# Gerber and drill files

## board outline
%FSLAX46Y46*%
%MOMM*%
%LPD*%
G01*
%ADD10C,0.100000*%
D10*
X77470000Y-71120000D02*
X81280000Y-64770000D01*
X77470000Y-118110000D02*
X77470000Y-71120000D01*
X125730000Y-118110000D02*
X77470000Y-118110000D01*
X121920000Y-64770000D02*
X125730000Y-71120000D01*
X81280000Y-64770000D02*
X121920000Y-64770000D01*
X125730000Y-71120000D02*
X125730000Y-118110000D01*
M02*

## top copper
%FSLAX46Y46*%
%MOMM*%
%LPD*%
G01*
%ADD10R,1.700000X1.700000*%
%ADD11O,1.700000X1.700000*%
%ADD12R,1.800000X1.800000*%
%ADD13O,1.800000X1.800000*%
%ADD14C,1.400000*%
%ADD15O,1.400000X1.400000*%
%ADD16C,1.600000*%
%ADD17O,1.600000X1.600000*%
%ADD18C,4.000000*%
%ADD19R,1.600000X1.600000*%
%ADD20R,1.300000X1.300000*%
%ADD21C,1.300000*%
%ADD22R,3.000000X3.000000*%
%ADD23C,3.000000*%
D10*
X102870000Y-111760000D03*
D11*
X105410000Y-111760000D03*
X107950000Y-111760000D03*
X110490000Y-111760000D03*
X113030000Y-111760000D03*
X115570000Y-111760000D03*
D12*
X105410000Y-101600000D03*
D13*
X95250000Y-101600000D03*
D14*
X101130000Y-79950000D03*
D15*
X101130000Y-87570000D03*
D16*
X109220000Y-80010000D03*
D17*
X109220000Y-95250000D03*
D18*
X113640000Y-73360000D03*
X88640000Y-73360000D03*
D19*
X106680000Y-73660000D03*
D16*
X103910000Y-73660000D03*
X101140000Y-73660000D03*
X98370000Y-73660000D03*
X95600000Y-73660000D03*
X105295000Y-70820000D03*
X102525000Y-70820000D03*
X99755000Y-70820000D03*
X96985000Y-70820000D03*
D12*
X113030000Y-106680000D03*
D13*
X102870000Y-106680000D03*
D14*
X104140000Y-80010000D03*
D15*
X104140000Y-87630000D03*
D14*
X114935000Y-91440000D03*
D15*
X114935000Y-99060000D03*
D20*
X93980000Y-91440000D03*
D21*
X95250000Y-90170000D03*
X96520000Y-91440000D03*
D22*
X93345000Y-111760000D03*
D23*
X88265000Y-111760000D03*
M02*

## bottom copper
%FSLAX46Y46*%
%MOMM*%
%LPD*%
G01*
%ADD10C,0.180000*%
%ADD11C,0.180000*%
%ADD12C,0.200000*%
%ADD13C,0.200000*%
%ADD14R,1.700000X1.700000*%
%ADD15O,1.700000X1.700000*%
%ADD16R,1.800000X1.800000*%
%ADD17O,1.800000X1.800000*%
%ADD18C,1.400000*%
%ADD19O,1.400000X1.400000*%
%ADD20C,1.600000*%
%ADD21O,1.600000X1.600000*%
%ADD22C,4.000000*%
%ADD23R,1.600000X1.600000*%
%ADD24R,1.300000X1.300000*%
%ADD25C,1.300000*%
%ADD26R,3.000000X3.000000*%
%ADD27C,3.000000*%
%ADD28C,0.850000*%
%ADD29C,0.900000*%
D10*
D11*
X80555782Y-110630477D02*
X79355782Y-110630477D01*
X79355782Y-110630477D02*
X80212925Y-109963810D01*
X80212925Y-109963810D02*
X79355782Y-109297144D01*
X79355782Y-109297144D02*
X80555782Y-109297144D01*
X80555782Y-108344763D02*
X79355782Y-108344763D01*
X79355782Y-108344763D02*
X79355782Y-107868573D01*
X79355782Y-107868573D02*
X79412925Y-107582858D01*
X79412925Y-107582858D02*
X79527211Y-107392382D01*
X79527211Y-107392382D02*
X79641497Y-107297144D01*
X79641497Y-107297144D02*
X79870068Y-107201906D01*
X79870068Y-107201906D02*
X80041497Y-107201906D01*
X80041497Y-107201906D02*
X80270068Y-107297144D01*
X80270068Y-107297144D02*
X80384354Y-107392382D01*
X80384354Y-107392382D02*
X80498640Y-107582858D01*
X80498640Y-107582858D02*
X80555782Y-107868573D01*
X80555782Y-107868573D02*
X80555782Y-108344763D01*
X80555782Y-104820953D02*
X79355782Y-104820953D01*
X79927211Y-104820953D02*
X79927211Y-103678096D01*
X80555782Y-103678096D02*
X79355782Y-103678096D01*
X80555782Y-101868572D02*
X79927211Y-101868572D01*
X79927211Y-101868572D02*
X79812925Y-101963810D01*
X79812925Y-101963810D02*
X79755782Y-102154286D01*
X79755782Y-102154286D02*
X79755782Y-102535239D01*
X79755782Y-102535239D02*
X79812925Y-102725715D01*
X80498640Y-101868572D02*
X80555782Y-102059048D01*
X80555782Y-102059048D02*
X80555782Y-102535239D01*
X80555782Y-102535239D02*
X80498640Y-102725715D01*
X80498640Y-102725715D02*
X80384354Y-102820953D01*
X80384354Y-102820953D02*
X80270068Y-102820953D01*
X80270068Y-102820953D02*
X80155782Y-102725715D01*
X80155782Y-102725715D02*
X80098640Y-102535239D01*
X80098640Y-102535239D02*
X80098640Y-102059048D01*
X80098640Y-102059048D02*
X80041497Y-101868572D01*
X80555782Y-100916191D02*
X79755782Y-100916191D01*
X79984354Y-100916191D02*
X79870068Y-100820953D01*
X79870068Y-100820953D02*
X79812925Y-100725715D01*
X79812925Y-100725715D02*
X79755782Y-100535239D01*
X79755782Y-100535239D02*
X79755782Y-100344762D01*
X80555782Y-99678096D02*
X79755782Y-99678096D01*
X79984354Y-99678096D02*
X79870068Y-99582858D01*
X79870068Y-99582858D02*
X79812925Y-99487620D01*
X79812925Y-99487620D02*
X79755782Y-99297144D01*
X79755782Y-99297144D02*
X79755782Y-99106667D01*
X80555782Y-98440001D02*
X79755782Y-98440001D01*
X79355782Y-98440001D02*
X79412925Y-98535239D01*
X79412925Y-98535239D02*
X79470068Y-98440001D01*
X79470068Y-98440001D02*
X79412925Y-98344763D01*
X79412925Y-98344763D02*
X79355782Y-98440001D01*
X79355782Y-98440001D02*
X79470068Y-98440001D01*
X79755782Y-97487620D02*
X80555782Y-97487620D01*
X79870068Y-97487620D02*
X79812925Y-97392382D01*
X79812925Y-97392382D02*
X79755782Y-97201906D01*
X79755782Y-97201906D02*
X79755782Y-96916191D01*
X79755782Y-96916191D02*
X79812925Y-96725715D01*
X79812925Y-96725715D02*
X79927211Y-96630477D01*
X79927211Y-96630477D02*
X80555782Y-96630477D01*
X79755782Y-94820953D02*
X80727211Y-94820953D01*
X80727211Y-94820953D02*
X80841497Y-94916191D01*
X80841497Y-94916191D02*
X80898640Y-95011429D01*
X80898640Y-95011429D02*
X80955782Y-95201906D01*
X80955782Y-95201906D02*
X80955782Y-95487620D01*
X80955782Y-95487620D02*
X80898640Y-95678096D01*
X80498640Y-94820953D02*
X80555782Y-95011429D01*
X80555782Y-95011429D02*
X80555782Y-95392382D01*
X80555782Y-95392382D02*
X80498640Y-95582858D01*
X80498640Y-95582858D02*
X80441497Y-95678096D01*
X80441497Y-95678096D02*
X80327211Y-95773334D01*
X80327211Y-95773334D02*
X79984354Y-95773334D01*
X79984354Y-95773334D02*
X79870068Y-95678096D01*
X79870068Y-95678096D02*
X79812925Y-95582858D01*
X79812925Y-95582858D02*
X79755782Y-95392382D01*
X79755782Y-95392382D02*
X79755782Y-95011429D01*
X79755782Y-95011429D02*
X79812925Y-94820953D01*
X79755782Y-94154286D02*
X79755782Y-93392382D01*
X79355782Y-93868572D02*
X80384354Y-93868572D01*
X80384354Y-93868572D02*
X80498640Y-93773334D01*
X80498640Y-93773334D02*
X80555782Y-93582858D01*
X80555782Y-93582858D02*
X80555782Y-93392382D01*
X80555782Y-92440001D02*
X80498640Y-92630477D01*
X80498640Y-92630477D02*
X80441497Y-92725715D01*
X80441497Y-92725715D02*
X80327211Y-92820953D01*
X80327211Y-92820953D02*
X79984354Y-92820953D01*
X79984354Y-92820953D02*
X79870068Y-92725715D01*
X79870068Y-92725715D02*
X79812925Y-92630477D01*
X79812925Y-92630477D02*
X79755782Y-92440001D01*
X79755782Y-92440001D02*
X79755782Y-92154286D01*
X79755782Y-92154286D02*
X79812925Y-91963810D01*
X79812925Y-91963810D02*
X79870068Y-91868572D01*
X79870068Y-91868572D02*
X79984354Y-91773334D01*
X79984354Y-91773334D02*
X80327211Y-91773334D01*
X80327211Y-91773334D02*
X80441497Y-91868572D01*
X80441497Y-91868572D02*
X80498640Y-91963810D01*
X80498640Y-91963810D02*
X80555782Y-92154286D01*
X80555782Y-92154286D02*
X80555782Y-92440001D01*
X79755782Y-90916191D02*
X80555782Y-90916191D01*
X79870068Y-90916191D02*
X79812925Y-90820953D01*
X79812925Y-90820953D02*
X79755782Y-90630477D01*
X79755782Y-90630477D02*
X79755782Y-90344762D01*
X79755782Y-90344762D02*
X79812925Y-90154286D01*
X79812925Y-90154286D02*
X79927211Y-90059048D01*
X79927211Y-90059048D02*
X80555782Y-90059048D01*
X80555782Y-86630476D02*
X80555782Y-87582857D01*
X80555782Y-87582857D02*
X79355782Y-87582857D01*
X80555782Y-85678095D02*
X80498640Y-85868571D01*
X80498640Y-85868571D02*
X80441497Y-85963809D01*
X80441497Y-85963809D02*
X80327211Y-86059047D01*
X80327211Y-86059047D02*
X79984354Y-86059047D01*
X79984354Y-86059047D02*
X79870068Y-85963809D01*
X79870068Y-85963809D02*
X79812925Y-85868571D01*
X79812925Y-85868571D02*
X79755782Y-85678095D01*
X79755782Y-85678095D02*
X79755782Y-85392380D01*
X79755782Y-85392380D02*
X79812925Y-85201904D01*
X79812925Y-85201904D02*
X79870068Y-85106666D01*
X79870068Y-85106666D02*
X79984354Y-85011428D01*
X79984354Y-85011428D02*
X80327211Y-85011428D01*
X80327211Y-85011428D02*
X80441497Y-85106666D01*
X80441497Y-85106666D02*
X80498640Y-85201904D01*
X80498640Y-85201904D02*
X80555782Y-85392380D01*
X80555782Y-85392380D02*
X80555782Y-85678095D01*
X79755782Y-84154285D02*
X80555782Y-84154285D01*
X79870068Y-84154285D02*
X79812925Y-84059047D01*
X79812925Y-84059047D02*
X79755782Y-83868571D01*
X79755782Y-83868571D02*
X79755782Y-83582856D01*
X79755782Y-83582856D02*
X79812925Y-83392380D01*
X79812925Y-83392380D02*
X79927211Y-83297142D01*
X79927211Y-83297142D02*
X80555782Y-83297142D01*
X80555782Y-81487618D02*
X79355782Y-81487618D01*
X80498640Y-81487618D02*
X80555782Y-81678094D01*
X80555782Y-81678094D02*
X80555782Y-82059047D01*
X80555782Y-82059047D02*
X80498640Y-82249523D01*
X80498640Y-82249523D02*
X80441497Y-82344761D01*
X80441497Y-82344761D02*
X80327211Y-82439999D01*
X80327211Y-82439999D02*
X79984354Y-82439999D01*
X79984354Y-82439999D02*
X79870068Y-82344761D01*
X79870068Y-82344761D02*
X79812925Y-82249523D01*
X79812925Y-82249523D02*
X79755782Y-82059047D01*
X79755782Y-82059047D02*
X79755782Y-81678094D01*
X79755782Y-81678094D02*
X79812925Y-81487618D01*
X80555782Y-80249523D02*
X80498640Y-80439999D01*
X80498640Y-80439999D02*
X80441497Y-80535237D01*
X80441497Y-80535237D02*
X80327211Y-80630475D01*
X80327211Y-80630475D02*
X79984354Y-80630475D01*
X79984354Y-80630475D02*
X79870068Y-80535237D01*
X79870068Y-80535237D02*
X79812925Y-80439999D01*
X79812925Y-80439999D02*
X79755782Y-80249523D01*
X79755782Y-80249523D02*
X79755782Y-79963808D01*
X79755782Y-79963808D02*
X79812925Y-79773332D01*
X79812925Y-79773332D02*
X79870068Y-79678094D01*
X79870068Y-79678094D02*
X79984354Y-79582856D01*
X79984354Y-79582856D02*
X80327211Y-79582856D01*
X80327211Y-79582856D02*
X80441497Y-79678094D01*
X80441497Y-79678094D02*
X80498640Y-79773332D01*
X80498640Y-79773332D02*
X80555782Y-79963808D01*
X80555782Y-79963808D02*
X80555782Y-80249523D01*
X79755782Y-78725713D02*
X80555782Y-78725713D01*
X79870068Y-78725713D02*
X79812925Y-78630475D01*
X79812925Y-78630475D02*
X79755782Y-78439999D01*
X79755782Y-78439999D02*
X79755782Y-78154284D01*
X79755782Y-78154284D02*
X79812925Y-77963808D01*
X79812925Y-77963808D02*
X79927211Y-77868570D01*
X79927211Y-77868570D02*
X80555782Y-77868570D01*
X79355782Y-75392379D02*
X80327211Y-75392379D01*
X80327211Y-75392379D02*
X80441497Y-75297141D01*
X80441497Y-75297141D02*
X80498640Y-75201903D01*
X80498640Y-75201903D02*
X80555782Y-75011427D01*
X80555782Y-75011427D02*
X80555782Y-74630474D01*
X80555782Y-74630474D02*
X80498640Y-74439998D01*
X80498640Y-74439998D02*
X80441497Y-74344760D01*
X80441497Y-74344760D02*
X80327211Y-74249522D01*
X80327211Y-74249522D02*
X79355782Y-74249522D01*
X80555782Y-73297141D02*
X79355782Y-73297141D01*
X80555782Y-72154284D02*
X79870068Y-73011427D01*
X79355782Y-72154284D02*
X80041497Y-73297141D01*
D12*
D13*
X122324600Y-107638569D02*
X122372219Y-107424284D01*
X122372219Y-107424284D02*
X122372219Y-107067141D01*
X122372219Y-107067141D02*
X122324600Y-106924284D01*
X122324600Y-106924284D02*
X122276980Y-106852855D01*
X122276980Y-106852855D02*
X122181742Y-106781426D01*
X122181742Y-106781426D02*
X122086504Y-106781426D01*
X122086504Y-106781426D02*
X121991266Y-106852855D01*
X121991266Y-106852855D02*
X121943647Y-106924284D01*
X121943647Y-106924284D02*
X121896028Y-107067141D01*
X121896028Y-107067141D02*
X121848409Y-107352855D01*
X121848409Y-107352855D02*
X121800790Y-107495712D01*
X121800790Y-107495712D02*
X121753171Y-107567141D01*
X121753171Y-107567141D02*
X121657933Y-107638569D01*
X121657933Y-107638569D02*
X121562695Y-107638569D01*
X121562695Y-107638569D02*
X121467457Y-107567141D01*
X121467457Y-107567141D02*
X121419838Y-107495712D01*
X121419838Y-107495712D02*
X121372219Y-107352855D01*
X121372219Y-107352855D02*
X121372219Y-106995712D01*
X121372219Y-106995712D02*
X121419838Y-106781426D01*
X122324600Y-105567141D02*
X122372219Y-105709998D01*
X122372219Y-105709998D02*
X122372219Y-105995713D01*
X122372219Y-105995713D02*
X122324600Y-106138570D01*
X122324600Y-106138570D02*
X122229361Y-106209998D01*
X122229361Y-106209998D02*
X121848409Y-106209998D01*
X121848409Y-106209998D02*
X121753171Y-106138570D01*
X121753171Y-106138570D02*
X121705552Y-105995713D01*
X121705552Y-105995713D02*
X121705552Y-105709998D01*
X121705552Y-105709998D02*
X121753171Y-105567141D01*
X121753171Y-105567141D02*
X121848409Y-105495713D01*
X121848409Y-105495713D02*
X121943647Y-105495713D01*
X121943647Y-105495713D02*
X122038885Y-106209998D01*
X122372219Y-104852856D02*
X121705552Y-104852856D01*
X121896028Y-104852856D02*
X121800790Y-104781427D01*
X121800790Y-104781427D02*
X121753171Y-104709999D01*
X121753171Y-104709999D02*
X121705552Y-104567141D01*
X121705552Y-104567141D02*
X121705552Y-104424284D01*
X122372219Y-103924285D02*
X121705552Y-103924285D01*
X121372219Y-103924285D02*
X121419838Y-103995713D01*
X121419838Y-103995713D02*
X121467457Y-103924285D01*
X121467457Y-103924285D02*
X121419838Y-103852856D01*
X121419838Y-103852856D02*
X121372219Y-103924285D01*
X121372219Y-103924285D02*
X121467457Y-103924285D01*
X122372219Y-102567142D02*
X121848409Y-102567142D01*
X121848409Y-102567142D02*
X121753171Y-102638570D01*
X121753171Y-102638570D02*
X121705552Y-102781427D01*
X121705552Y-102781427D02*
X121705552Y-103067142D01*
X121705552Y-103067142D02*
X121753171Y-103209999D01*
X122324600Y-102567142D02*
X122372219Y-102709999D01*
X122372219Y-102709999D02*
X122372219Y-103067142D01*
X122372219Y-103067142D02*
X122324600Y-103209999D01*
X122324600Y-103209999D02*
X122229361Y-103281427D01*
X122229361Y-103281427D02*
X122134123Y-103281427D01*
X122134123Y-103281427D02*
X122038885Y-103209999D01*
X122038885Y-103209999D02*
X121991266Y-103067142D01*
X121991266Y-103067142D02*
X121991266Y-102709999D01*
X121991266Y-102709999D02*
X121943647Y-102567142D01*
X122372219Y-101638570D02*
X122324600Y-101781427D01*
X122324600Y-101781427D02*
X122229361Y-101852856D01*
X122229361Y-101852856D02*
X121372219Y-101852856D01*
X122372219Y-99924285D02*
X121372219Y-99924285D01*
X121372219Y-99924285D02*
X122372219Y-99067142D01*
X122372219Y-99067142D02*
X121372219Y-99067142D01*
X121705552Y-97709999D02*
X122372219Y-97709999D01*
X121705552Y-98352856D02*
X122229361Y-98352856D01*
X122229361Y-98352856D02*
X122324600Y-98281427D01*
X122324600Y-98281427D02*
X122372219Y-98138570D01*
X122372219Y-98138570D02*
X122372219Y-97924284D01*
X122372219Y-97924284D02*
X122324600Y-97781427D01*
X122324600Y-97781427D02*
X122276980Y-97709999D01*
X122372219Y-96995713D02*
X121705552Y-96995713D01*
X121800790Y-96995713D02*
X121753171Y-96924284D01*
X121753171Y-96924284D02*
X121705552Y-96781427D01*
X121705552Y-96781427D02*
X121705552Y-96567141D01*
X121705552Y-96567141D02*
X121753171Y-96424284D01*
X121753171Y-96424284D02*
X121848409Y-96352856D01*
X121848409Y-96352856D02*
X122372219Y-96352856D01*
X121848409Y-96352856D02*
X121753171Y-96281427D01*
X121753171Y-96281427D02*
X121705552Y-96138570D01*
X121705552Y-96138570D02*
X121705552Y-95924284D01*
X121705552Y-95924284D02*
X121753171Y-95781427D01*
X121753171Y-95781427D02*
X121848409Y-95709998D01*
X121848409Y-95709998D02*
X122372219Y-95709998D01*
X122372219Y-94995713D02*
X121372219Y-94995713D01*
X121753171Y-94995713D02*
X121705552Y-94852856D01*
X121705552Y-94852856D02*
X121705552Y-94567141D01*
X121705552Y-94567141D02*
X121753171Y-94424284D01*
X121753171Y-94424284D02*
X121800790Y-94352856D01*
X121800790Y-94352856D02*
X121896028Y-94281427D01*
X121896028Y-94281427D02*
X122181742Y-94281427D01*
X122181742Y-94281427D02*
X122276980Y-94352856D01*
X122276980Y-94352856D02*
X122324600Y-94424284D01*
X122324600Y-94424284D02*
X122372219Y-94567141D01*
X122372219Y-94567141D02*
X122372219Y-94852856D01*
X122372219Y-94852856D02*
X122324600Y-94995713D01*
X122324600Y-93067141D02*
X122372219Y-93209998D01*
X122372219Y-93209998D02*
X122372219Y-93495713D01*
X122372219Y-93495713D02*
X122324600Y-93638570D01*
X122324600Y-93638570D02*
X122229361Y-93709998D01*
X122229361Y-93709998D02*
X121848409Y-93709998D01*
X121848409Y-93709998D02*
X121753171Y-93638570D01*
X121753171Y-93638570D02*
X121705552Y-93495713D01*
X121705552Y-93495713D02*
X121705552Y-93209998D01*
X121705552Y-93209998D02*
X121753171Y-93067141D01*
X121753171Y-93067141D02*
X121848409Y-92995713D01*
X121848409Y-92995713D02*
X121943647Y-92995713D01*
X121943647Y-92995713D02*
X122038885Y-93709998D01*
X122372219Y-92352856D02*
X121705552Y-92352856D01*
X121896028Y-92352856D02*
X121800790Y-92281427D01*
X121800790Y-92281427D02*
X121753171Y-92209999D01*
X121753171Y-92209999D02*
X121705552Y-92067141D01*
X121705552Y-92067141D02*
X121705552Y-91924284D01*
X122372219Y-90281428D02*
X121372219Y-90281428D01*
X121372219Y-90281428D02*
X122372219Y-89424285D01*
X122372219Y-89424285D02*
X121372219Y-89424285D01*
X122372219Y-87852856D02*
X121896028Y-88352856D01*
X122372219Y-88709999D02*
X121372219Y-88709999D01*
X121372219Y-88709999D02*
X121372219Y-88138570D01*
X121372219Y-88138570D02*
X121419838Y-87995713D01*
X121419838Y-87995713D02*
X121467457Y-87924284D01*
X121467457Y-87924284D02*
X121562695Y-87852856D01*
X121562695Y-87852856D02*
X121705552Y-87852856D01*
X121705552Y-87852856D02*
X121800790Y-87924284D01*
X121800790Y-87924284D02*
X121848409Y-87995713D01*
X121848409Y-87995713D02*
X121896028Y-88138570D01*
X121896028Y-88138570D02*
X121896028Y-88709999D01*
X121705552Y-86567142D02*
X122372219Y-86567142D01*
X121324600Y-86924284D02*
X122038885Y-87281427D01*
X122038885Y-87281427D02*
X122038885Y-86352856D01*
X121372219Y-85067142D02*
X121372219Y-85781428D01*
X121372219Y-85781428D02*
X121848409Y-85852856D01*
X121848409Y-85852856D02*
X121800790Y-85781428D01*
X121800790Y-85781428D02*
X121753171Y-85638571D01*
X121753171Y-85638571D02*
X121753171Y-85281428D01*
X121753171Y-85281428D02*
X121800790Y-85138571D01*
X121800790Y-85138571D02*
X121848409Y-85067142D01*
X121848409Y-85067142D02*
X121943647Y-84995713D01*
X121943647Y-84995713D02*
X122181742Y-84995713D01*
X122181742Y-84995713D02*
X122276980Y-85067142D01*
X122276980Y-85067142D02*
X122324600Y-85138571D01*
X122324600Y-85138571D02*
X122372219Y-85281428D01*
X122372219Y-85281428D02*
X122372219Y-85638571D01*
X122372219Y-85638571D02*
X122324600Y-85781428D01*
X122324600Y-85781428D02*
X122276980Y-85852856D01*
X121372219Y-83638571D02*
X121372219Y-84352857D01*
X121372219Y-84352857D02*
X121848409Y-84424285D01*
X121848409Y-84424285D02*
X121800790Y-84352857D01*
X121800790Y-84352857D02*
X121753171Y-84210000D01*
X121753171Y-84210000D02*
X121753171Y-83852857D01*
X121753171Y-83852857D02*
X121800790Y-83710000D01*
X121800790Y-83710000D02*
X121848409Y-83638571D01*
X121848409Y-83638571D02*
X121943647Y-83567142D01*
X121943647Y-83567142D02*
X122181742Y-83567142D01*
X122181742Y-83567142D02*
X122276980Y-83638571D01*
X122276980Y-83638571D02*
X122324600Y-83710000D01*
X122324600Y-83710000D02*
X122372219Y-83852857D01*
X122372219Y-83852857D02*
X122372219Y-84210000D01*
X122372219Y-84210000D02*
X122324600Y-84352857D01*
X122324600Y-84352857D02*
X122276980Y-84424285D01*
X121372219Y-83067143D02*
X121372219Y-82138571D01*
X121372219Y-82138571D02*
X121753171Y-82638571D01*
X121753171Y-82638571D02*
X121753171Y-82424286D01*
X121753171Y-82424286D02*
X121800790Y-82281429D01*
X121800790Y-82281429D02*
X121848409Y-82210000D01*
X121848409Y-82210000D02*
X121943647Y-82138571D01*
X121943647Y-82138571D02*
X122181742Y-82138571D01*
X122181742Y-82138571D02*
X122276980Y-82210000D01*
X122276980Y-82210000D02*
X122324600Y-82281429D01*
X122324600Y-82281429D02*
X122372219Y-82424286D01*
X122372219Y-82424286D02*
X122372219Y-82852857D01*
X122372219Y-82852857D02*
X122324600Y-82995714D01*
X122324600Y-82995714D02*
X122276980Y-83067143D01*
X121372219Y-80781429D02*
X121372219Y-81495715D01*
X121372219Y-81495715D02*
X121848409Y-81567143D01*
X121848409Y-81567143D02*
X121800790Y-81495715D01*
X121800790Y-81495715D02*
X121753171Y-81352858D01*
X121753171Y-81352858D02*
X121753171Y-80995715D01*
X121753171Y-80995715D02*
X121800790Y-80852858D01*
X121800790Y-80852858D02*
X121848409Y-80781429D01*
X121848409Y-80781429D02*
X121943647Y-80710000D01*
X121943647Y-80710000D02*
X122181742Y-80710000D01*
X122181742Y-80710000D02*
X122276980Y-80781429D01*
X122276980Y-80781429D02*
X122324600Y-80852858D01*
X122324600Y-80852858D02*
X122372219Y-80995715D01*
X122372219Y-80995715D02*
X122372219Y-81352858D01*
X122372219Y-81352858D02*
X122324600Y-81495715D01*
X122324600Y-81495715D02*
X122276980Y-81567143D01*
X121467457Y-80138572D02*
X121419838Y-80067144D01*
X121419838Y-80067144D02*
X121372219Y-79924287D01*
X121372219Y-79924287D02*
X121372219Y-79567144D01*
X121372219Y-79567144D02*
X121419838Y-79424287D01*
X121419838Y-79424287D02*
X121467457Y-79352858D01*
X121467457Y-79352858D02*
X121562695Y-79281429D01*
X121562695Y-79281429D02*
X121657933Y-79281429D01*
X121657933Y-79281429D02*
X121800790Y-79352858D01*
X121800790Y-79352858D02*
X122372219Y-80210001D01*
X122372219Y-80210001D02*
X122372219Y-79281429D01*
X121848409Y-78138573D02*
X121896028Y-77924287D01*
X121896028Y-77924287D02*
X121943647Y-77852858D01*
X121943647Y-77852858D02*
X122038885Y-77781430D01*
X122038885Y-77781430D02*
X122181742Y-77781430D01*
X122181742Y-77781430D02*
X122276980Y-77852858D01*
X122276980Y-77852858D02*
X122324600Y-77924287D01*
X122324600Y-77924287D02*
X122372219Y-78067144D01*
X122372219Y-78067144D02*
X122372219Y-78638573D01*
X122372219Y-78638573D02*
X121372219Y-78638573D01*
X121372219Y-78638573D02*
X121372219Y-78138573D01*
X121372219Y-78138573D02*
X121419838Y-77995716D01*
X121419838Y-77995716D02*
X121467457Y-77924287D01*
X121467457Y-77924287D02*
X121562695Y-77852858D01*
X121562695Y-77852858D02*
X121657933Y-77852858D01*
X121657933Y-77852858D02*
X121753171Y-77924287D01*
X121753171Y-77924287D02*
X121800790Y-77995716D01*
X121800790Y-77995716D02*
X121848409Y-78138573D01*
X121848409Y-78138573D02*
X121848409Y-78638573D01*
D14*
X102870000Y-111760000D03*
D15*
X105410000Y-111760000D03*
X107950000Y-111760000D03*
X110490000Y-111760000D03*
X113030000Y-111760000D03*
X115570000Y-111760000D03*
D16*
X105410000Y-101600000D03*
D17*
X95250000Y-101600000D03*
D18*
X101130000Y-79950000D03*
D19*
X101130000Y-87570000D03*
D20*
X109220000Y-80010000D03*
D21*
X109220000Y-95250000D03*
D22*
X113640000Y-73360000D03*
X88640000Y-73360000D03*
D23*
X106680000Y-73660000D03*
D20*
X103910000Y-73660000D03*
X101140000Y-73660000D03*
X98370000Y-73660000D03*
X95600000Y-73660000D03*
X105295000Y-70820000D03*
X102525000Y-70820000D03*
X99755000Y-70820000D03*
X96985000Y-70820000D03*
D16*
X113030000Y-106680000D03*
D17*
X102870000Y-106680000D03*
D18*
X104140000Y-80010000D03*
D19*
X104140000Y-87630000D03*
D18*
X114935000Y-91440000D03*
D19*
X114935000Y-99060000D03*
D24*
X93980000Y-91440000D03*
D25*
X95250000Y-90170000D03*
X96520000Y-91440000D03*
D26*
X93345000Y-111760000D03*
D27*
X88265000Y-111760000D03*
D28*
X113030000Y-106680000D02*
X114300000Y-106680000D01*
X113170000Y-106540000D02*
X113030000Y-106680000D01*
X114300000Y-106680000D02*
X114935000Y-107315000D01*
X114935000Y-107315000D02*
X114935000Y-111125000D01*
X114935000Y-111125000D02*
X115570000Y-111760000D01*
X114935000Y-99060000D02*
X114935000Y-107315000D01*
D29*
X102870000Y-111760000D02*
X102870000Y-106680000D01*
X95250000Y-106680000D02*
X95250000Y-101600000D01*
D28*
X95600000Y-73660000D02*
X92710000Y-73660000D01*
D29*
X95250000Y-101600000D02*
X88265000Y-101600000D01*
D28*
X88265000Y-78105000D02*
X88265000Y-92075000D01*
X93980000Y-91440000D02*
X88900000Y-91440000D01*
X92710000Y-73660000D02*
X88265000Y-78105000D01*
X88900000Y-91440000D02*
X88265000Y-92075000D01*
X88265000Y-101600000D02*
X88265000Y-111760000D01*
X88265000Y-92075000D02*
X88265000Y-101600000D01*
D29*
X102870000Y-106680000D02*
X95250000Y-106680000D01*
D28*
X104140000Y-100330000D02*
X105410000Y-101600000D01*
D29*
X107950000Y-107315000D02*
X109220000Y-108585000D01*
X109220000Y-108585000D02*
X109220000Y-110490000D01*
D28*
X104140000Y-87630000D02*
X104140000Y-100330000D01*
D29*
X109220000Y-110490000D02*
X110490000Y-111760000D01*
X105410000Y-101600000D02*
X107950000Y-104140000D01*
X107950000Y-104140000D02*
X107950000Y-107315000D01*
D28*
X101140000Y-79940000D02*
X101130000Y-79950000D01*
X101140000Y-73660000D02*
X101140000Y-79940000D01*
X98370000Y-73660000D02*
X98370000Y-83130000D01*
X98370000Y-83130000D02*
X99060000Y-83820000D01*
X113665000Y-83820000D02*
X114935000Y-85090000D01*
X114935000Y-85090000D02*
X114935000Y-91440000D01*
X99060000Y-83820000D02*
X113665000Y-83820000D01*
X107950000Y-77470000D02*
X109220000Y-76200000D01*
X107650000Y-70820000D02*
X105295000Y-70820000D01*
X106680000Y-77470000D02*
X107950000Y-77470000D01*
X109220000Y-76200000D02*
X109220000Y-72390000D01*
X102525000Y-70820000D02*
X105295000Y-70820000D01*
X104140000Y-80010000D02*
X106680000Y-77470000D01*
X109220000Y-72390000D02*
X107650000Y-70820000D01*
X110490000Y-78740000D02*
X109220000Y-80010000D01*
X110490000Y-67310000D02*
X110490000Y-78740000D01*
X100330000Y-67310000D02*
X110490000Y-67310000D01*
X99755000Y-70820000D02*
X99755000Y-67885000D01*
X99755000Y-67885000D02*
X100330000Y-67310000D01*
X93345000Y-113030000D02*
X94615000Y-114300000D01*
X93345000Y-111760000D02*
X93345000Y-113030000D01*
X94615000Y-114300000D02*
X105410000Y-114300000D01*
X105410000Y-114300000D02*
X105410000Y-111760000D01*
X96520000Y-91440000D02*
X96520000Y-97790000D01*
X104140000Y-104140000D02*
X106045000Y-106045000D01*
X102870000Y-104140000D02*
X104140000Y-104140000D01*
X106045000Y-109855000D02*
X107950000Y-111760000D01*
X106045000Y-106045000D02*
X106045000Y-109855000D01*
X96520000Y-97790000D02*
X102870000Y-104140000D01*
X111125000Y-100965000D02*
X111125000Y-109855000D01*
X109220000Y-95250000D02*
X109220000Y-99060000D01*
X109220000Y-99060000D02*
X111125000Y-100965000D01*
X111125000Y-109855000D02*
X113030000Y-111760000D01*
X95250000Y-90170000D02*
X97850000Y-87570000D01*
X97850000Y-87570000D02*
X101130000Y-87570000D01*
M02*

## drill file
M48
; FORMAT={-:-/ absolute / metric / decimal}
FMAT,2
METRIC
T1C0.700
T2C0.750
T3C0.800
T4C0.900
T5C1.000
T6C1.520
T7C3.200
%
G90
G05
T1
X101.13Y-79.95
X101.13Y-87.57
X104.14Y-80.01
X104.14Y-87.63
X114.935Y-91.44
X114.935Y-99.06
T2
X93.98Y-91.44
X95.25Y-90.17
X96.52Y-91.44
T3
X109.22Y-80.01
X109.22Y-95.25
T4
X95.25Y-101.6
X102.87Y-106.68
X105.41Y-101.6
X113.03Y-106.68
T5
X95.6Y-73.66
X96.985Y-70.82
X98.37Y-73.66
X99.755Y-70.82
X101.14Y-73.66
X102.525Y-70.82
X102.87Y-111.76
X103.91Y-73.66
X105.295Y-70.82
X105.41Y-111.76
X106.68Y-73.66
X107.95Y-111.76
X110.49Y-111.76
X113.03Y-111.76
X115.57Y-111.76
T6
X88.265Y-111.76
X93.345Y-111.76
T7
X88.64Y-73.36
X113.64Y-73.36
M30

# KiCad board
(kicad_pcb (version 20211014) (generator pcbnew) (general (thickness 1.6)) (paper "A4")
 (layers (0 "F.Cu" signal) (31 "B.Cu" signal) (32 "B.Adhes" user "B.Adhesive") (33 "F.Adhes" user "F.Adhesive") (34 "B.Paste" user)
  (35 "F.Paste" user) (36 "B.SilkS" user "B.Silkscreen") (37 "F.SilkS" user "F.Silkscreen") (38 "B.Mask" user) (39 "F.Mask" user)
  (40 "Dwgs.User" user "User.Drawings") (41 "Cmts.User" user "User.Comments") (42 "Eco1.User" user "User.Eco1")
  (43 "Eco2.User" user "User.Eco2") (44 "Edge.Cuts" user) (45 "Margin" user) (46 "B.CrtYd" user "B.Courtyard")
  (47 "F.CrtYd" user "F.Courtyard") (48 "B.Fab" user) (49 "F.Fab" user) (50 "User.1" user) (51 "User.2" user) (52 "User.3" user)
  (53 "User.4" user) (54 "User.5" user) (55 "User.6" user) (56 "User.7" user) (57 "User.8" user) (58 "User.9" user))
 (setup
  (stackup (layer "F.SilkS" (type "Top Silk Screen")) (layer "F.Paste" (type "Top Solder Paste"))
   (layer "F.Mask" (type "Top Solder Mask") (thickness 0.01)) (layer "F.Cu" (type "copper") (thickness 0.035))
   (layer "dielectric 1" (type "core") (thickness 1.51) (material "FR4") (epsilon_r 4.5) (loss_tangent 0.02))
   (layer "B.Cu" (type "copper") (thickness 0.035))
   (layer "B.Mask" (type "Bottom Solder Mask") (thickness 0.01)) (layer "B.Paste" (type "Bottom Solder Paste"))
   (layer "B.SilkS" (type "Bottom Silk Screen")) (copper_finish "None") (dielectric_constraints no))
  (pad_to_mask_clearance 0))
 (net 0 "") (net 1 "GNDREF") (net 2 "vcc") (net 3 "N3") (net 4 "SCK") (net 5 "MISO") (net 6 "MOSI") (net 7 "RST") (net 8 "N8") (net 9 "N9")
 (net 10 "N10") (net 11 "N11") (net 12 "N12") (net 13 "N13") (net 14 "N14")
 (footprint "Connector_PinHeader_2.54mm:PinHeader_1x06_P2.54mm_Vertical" (layer "F.Cu") (at 102.87 111.76 90)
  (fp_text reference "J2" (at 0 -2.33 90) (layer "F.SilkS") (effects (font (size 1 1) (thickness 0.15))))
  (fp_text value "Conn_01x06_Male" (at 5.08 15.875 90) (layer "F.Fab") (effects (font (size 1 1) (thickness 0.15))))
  (pad "1" thru_hole rect (at 0 0 90) (size 1.7 1.7) (drill 1) (layers *.Cu *.Mask) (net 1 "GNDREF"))
  (pad "2" thru_hole oval (at 0 2.54 90) (size 1.7 1.7) (drill 1) (layers *.Cu *.Mask) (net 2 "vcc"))
  (pad "3" thru_hole oval (at 0 5.08 90) (size 1.7 1.7) (drill 1) (layers *.Cu *.Mask) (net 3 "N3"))
  (pad "4" thru_hole oval (at 0 7.62 90) (size 1.7 1.7) (drill 1) (layers *.Cu *.Mask) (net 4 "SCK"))
  (pad "5" thru_hole oval (at 0 10.16 90) (size 1.7 1.7) (drill 1) (layers *.Cu *.Mask) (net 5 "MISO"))
  (pad "6" thru_hole oval (at 0 12.7 90) (size 1.7 1.7) (drill 1) (layers *.Cu *.Mask) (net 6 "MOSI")))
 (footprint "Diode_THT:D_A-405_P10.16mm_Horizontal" (layer "F.Cu") (at 105.41 101.6 180)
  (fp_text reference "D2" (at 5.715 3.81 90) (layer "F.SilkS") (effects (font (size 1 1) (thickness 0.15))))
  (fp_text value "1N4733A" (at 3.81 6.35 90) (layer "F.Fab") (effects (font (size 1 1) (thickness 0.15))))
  (pad "1" thru_hole rect (at 0 0 180) (size 1.8 1.8) (drill 0.9) (layers *.Cu *.Mask) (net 4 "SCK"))
  (pad "2" thru_hole oval (at 10.16 0 180) (size 1.8 1.8) (drill 0.9) (layers *.Cu *.Mask) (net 1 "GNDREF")))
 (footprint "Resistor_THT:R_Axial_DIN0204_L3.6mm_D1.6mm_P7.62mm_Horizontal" (layer "F.Cu") (at 101.13 79.95 -90)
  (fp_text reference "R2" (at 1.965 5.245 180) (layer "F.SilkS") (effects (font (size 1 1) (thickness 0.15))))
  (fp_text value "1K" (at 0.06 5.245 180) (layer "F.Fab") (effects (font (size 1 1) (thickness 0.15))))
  (pad "1" thru_hole circle (at 0 0 270) (size 1.4 1.4) (drill 0.7) (layers *.Cu *.Mask) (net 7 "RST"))
  (pad "2" thru_hole oval (at 7.62 0 270) (size 1.4 1.4) (drill 0.7) (layers *.Cu *.Mask) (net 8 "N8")))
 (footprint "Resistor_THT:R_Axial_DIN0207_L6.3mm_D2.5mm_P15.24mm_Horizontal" (layer "F.Cu") (at 109.22 80.01 -90)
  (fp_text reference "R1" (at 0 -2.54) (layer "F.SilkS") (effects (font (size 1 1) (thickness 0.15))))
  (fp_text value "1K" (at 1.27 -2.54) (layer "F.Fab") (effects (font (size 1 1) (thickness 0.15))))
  (pad "1" thru_hole circle (at 0 0 270) (size 1.6 1.6) (drill 0.8) (layers *.Cu *.Mask) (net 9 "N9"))
  (pad "2" thru_hole oval (at 15.24 0 270) (size 1.6 1.6) (drill 0.8) (layers *.Cu *.Mask) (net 5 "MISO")))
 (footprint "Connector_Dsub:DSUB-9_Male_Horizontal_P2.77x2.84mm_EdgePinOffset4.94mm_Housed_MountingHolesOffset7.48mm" (layer "F.Cu")
  (at 106.68 73.66 180)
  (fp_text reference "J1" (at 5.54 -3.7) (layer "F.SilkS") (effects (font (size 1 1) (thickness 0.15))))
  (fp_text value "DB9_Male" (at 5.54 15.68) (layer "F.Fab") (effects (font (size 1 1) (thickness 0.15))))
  (pad "0" thru_hole circle (at -6.96 0.3 180) (size 4 4) (drill 3.2) (layers *.Cu *.Mask))
  (pad "0" thru_hole circle (at 18.04 0.3 180) (size 4 4) (drill 3.2) (layers *.Cu *.Mask))
  (pad "1" thru_hole rect (at 0 0 180) (size 1.6 1.6) (drill 1) (layers *.Cu *.Mask) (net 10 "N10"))
  (pad "2" thru_hole circle (at 2.77 0 180) (size 1.6 1.6) (drill 1) (layers *.Cu *.Mask) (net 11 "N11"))
  (pad "3" thru_hole circle (at 5.54 0 180) (size 1.6 1.6) (drill 1) (layers *.Cu *.Mask) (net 7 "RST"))
  (pad "4" thru_hole circle (at 8.31 0 180) (size 1.6 1.6) (drill 1) (layers *.Cu *.Mask) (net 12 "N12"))
  (pad "5" thru_hole circle (at 11.08 0 180) (size 1.6 1.6) (drill 1) (layers *.Cu *.Mask) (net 1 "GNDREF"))
  (pad "6" thru_hole circle (at 1.385 2.84 180) (size 1.6 1.6) (drill 1) (layers *.Cu *.Mask) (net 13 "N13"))
  (pad "7" thru_hole circle (at 4.155 2.84 180) (size 1.6 1.6) (drill 1) (layers *.Cu *.Mask) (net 13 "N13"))
  (pad "8" thru_hole circle (at 6.925 2.84 180) (size 1.6 1.6) (drill 1) (layers *.Cu *.Mask) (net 9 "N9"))
  (pad "9" thru_hole circle (at 9.695 2.84 180) (size 1.6 1.6) (drill 1) (layers *.Cu *.Mask) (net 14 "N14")))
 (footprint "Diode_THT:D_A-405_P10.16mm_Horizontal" (layer "F.Cu") (at 113.03 106.68 180)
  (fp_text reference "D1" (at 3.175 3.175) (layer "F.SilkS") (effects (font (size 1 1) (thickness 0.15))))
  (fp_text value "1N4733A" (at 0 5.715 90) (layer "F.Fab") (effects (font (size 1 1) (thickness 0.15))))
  (pad "1" thru_hole rect (at 0 0 180) (size 1.8 1.8) (drill 0.9) (layers *.Cu *.Mask) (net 6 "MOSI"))
  (pad "2" thru_hole oval (at 10.16 0 180) (size 1.8 1.8) (drill 0.9) (layers *.Cu *.Mask) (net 1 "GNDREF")))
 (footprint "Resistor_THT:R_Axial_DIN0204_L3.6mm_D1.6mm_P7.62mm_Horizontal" (layer "F.Cu") (at 104.14 80.01 -90)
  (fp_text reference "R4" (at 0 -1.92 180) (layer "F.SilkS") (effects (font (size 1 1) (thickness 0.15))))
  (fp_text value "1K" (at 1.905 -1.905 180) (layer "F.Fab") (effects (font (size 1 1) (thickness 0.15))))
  (pad "1" thru_hole circle (at 0 0 270) (size 1.4 1.4) (drill 0.7) (layers *.Cu *.Mask) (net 13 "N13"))
  (pad "2" thru_hole oval (at 7.62 0 270) (size 1.4 1.4) (drill 0.7) (layers *.Cu *.Mask) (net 4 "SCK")))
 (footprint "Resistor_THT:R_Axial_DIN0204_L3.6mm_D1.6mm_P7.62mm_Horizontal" (layer "F.Cu") (at 114.935 91.44 -90)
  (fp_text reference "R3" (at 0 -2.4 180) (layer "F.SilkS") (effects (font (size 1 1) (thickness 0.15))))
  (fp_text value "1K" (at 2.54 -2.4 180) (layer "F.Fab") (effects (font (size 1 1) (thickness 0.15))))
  (pad "1" thru_hole circle (at 0 0 270) (size 1.4 1.4) (drill 0.7) (layers *.Cu *.Mask) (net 12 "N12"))
  (pad "2" thru_hole oval (at 7.62 0 270) (size 1.4 1.4) (drill 0.7) (layers *.Cu *.Mask) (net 6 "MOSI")))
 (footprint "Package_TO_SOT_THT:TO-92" (layer "F.Cu") (at 93.98 91.44)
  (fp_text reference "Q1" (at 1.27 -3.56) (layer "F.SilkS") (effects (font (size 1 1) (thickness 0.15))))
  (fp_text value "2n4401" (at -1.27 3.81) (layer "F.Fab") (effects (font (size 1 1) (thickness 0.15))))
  (pad "1" thru_hole rect (at 0 0) (size 1.3 1.3) (drill 0.75) (layers *.Cu *.Mask) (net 1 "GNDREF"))
  (pad "2" thru_hole circle (at 1.27 -1.27) (size 1.3 1.3) (drill 0.75) (layers *.Cu *.Mask) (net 8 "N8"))
  (pad "3" thru_hole circle (at 2.54 0) (size 1.3 1.3) (drill 0.75) (layers *.Cu *.Mask) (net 3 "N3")))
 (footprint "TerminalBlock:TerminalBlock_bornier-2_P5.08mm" (layer "F.Cu") (at 93.345 111.76 180)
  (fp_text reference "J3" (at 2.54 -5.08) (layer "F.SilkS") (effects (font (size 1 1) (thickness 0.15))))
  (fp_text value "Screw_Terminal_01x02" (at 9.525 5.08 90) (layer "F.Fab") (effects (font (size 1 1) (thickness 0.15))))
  (pad "1" thru_hole rect (at 0 0 180) (size 3 3) (drill 1.52) (layers *.Cu *.Mask) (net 2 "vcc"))
  (pad "2" thru_hole circle (at 5.08 0 180) (size 3 3) (drill 1.52) (layers *.Cu *.Mask) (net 1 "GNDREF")))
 (gr_line (start 77.47 71.12) (end 81.28 64.77) (layer "Edge.Cuts") (width 0.1))
 (gr_line (start 77.47 118.11) (end 77.47 71.12) (layer "Edge.Cuts") (width 0.1))
 (gr_line (start 125.73 118.11) (end 77.47 118.11) (layer "Edge.Cuts") (width 0.1))
 (gr_line (start 121.92 64.77) (end 125.73 71.12) (layer "Edge.Cuts") (width 0.1))
 (gr_line (start 81.28 64.77) (end 121.92 64.77) (layer "Edge.Cuts") (width 0.1))
 (gr_line (start 125.73 71.12) (end 125.73 118.11) (layer "Edge.Cuts") (width 0.1))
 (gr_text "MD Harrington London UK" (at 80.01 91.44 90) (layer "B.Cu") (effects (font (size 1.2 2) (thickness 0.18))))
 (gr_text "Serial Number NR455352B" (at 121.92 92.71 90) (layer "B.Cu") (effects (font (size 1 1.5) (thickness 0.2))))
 (segment (start 113.03 106.68) (end 114.3 106.68) (width 0.85) (layer "B.Cu") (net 6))
 (segment (start 113.17 106.54) (end 113.03 106.68) (width 0.85) (layer "B.Cu") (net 6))
 (segment (start 114.3 106.68) (end 114.935 107.315) (width 0.85) (layer "B.Cu") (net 6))
 (segment (start 114.935 107.315) (end 114.935 111.125) (width 0.85) (layer "B.Cu") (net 6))
 (segment (start 114.935 111.125) (end 115.57 111.76) (width 0.85) (layer "B.Cu") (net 6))
 (segment (start 114.935 99.06) (end 114.935 107.315) (width 0.85) (layer "B.Cu") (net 6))
 (segment (start 102.87 111.76) (end 102.87 106.68) (width 0.9) (layer "B.Cu") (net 1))
 (segment (start 95.25 106.68) (end 95.25 101.6) (width 0.9) (layer "B.Cu") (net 1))
 (segment (start 95.6 73.66) (end 92.71 73.66) (width 0.85) (layer "B.Cu") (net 1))
 (segment (start 95.25 101.6) (end 88.265 101.6) (width 0.9) (layer "B.Cu") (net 1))
 (segment (start 88.265 78.105) (end 88.265 92.075) (width 0.85) (layer "B.Cu") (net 1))
 (segment (start 93.98 91.44) (end 88.9 91.44) (width 0.85) (layer "B.Cu") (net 1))
 (segment (start 92.71 73.66) (end 88.265 78.105) (width 0.85) (layer "B.Cu") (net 1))
 (segment (start 88.9 91.44) (end 88.265 92.075) (width 0.85) (layer "B.Cu") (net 1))
 (segment (start 88.265 101.6) (end 88.265 111.76) (width 0.85) (layer "B.Cu") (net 1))
 (segment (start 88.265 92.075) (end 88.265 101.6) (width 0.85) (layer "B.Cu") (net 1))
 (segment (start 102.87 106.68) (end 95.25 106.68) (width 0.9) (layer "B.Cu") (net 1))
 (segment (start 104.14 100.33) (end 105.41 101.6) (width 0.85) (layer "B.Cu") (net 4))
 (segment (start 107.95 107.315) (end 109.22 108.585) (width 0.9) (layer "B.Cu") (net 4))
 (segment (start 109.22 108.585) (end 109.22 110.49) (width 0.9) (layer "B.Cu") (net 4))
 (segment (start 104.14 87.63) (end 104.14 100.33) (width 0.85) (layer "B.Cu") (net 4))
 (segment (start 109.22 110.49) (end 110.49 111.76) (width 0.9) (layer "B.Cu") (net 4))
 (segment (start 105.41 101.6) (end 107.95 104.14) (width 0.9) (layer "B.Cu") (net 4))
 (segment (start 107.95 104.14) (end 107.95 107.315) (width 0.9) (layer "B.Cu") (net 4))
 (segment (start 101.14 79.94) (end 101.13 79.95) (width 0.85) (layer "B.Cu") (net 7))
 (segment (start 101.14 73.66) (end 101.14 79.94) (width 0.85) (layer "B.Cu") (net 7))
 (segment (start 98.37 73.66) (end 98.37 83.13) (width 0.85) (layer "B.Cu") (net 12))
 (segment (start 98.37 83.13) (end 99.06 83.82) (width 0.85) (layer "B.Cu") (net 12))
 (segment (start 113.665 83.82) (end 114.935 85.09) (width 0.85) (layer "B.Cu") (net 12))
 (segment (start 114.935 85.09) (end 114.935 91.44) (width 0.85) (layer "B.Cu") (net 12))
 (segment (start 99.06 83.82) (end 113.665 83.82) (width 0.85) (layer "B.Cu") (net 12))
 (segment (start 107.95 77.47) (end 109.22 76.2) (width 0.85) (layer "B.Cu") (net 13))
 (segment (start 107.65 70.82) (end 105.295 70.82) (width 0.85) (layer "B.Cu") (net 13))
 (segment (start 106.68 77.47) (end 107.95 77.47) (width 0.85) (layer "B.Cu") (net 13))
 (segment (start 109.22 76.2) (end 109.22 72.39) (width 0.85) (layer "B.Cu") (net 13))
 (segment (start 102.525 70.82) (end 105.295 70.82) (width 0.85) (layer "B.Cu") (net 13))
 (segment (start 104.14 80.01) (end 106.68 77.47) (width 0.85) (layer "B.Cu") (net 13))
 (segment (start 109.22 72.39) (end 107.65 70.82) (width 0.85) (layer "B.Cu") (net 13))
 (segment (start 110.49 78.74) (end 109.22 80.01) (width 0.85) (layer "B.Cu") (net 9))
 (segment (start 110.49 67.31) (end 110.49 78.74) (width 0.85) (layer "B.Cu") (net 9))
 (segment (start 100.33 67.31) (end 110.49 67.31) (width 0.85) (layer "B.Cu") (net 9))
 (segment (start 99.755 70.82) (end 99.755 67.885) (width 0.85) (layer "B.Cu") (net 9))
 (segment (start 99.755 67.885) (end 100.33 67.31) (width 0.85) (layer "B.Cu") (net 9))
 (segment (start 93.345 113.03) (end 94.615 114.3) (width 0.85) (layer "B.Cu") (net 2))
 (segment (start 93.345 111.76) (end 93.345 113.03) (width 0.85) (layer "B.Cu") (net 2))
 (segment (start 94.615 114.3) (end 105.41 114.3) (width 0.85) (layer "B.Cu") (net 2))
 (segment (start 105.41 114.3) (end 105.41 111.76) (width 0.85) (layer "B.Cu") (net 2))
 (segment (start 96.52 91.44) (end 96.52 97.79) (width 0.85) (layer "B.Cu") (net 3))
 (segment (start 104.14 104.14) (end 106.045 106.045) (width 0.85) (layer "B.Cu") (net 3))
 (segment (start 102.87 104.14) (end 104.14 104.14) (width 0.85) (layer "B.Cu") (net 3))
 (segment (start 106.045 109.855) (end 107.95 111.76) (width 0.85) (layer "B.Cu") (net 3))
 (segment (start 106.045 106.045) (end 106.045 109.855) (width 0.85) (layer "B.Cu") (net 3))
 (segment (start 96.52 97.79) (end 102.87 104.14) (width 0.85) (layer "B.Cu") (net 3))
 (segment (start 111.125 100.965) (end 111.125 109.855) (width 0.85) (layer "B.Cu") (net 5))
 (segment (start 109.22 95.25) (end 109.22 99.06) (width 0.85) (layer "B.Cu") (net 5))
 (segment (start 109.22 99.06) (end 111.125 100.965) (width 0.85) (layer "B.Cu") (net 5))
 (segment (start 111.125 109.855) (end 113.03 111.76) (width 0.85) (layer "B.Cu") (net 5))
 (segment (start 95.25 90.17) (end 97.85 87.57) (width 0.85) (layer "B.Cu") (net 8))
 (segment (start 97.85 87.57) (end 101.13 87.57) (width 0.85) (layer "B.Cu") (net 8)))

